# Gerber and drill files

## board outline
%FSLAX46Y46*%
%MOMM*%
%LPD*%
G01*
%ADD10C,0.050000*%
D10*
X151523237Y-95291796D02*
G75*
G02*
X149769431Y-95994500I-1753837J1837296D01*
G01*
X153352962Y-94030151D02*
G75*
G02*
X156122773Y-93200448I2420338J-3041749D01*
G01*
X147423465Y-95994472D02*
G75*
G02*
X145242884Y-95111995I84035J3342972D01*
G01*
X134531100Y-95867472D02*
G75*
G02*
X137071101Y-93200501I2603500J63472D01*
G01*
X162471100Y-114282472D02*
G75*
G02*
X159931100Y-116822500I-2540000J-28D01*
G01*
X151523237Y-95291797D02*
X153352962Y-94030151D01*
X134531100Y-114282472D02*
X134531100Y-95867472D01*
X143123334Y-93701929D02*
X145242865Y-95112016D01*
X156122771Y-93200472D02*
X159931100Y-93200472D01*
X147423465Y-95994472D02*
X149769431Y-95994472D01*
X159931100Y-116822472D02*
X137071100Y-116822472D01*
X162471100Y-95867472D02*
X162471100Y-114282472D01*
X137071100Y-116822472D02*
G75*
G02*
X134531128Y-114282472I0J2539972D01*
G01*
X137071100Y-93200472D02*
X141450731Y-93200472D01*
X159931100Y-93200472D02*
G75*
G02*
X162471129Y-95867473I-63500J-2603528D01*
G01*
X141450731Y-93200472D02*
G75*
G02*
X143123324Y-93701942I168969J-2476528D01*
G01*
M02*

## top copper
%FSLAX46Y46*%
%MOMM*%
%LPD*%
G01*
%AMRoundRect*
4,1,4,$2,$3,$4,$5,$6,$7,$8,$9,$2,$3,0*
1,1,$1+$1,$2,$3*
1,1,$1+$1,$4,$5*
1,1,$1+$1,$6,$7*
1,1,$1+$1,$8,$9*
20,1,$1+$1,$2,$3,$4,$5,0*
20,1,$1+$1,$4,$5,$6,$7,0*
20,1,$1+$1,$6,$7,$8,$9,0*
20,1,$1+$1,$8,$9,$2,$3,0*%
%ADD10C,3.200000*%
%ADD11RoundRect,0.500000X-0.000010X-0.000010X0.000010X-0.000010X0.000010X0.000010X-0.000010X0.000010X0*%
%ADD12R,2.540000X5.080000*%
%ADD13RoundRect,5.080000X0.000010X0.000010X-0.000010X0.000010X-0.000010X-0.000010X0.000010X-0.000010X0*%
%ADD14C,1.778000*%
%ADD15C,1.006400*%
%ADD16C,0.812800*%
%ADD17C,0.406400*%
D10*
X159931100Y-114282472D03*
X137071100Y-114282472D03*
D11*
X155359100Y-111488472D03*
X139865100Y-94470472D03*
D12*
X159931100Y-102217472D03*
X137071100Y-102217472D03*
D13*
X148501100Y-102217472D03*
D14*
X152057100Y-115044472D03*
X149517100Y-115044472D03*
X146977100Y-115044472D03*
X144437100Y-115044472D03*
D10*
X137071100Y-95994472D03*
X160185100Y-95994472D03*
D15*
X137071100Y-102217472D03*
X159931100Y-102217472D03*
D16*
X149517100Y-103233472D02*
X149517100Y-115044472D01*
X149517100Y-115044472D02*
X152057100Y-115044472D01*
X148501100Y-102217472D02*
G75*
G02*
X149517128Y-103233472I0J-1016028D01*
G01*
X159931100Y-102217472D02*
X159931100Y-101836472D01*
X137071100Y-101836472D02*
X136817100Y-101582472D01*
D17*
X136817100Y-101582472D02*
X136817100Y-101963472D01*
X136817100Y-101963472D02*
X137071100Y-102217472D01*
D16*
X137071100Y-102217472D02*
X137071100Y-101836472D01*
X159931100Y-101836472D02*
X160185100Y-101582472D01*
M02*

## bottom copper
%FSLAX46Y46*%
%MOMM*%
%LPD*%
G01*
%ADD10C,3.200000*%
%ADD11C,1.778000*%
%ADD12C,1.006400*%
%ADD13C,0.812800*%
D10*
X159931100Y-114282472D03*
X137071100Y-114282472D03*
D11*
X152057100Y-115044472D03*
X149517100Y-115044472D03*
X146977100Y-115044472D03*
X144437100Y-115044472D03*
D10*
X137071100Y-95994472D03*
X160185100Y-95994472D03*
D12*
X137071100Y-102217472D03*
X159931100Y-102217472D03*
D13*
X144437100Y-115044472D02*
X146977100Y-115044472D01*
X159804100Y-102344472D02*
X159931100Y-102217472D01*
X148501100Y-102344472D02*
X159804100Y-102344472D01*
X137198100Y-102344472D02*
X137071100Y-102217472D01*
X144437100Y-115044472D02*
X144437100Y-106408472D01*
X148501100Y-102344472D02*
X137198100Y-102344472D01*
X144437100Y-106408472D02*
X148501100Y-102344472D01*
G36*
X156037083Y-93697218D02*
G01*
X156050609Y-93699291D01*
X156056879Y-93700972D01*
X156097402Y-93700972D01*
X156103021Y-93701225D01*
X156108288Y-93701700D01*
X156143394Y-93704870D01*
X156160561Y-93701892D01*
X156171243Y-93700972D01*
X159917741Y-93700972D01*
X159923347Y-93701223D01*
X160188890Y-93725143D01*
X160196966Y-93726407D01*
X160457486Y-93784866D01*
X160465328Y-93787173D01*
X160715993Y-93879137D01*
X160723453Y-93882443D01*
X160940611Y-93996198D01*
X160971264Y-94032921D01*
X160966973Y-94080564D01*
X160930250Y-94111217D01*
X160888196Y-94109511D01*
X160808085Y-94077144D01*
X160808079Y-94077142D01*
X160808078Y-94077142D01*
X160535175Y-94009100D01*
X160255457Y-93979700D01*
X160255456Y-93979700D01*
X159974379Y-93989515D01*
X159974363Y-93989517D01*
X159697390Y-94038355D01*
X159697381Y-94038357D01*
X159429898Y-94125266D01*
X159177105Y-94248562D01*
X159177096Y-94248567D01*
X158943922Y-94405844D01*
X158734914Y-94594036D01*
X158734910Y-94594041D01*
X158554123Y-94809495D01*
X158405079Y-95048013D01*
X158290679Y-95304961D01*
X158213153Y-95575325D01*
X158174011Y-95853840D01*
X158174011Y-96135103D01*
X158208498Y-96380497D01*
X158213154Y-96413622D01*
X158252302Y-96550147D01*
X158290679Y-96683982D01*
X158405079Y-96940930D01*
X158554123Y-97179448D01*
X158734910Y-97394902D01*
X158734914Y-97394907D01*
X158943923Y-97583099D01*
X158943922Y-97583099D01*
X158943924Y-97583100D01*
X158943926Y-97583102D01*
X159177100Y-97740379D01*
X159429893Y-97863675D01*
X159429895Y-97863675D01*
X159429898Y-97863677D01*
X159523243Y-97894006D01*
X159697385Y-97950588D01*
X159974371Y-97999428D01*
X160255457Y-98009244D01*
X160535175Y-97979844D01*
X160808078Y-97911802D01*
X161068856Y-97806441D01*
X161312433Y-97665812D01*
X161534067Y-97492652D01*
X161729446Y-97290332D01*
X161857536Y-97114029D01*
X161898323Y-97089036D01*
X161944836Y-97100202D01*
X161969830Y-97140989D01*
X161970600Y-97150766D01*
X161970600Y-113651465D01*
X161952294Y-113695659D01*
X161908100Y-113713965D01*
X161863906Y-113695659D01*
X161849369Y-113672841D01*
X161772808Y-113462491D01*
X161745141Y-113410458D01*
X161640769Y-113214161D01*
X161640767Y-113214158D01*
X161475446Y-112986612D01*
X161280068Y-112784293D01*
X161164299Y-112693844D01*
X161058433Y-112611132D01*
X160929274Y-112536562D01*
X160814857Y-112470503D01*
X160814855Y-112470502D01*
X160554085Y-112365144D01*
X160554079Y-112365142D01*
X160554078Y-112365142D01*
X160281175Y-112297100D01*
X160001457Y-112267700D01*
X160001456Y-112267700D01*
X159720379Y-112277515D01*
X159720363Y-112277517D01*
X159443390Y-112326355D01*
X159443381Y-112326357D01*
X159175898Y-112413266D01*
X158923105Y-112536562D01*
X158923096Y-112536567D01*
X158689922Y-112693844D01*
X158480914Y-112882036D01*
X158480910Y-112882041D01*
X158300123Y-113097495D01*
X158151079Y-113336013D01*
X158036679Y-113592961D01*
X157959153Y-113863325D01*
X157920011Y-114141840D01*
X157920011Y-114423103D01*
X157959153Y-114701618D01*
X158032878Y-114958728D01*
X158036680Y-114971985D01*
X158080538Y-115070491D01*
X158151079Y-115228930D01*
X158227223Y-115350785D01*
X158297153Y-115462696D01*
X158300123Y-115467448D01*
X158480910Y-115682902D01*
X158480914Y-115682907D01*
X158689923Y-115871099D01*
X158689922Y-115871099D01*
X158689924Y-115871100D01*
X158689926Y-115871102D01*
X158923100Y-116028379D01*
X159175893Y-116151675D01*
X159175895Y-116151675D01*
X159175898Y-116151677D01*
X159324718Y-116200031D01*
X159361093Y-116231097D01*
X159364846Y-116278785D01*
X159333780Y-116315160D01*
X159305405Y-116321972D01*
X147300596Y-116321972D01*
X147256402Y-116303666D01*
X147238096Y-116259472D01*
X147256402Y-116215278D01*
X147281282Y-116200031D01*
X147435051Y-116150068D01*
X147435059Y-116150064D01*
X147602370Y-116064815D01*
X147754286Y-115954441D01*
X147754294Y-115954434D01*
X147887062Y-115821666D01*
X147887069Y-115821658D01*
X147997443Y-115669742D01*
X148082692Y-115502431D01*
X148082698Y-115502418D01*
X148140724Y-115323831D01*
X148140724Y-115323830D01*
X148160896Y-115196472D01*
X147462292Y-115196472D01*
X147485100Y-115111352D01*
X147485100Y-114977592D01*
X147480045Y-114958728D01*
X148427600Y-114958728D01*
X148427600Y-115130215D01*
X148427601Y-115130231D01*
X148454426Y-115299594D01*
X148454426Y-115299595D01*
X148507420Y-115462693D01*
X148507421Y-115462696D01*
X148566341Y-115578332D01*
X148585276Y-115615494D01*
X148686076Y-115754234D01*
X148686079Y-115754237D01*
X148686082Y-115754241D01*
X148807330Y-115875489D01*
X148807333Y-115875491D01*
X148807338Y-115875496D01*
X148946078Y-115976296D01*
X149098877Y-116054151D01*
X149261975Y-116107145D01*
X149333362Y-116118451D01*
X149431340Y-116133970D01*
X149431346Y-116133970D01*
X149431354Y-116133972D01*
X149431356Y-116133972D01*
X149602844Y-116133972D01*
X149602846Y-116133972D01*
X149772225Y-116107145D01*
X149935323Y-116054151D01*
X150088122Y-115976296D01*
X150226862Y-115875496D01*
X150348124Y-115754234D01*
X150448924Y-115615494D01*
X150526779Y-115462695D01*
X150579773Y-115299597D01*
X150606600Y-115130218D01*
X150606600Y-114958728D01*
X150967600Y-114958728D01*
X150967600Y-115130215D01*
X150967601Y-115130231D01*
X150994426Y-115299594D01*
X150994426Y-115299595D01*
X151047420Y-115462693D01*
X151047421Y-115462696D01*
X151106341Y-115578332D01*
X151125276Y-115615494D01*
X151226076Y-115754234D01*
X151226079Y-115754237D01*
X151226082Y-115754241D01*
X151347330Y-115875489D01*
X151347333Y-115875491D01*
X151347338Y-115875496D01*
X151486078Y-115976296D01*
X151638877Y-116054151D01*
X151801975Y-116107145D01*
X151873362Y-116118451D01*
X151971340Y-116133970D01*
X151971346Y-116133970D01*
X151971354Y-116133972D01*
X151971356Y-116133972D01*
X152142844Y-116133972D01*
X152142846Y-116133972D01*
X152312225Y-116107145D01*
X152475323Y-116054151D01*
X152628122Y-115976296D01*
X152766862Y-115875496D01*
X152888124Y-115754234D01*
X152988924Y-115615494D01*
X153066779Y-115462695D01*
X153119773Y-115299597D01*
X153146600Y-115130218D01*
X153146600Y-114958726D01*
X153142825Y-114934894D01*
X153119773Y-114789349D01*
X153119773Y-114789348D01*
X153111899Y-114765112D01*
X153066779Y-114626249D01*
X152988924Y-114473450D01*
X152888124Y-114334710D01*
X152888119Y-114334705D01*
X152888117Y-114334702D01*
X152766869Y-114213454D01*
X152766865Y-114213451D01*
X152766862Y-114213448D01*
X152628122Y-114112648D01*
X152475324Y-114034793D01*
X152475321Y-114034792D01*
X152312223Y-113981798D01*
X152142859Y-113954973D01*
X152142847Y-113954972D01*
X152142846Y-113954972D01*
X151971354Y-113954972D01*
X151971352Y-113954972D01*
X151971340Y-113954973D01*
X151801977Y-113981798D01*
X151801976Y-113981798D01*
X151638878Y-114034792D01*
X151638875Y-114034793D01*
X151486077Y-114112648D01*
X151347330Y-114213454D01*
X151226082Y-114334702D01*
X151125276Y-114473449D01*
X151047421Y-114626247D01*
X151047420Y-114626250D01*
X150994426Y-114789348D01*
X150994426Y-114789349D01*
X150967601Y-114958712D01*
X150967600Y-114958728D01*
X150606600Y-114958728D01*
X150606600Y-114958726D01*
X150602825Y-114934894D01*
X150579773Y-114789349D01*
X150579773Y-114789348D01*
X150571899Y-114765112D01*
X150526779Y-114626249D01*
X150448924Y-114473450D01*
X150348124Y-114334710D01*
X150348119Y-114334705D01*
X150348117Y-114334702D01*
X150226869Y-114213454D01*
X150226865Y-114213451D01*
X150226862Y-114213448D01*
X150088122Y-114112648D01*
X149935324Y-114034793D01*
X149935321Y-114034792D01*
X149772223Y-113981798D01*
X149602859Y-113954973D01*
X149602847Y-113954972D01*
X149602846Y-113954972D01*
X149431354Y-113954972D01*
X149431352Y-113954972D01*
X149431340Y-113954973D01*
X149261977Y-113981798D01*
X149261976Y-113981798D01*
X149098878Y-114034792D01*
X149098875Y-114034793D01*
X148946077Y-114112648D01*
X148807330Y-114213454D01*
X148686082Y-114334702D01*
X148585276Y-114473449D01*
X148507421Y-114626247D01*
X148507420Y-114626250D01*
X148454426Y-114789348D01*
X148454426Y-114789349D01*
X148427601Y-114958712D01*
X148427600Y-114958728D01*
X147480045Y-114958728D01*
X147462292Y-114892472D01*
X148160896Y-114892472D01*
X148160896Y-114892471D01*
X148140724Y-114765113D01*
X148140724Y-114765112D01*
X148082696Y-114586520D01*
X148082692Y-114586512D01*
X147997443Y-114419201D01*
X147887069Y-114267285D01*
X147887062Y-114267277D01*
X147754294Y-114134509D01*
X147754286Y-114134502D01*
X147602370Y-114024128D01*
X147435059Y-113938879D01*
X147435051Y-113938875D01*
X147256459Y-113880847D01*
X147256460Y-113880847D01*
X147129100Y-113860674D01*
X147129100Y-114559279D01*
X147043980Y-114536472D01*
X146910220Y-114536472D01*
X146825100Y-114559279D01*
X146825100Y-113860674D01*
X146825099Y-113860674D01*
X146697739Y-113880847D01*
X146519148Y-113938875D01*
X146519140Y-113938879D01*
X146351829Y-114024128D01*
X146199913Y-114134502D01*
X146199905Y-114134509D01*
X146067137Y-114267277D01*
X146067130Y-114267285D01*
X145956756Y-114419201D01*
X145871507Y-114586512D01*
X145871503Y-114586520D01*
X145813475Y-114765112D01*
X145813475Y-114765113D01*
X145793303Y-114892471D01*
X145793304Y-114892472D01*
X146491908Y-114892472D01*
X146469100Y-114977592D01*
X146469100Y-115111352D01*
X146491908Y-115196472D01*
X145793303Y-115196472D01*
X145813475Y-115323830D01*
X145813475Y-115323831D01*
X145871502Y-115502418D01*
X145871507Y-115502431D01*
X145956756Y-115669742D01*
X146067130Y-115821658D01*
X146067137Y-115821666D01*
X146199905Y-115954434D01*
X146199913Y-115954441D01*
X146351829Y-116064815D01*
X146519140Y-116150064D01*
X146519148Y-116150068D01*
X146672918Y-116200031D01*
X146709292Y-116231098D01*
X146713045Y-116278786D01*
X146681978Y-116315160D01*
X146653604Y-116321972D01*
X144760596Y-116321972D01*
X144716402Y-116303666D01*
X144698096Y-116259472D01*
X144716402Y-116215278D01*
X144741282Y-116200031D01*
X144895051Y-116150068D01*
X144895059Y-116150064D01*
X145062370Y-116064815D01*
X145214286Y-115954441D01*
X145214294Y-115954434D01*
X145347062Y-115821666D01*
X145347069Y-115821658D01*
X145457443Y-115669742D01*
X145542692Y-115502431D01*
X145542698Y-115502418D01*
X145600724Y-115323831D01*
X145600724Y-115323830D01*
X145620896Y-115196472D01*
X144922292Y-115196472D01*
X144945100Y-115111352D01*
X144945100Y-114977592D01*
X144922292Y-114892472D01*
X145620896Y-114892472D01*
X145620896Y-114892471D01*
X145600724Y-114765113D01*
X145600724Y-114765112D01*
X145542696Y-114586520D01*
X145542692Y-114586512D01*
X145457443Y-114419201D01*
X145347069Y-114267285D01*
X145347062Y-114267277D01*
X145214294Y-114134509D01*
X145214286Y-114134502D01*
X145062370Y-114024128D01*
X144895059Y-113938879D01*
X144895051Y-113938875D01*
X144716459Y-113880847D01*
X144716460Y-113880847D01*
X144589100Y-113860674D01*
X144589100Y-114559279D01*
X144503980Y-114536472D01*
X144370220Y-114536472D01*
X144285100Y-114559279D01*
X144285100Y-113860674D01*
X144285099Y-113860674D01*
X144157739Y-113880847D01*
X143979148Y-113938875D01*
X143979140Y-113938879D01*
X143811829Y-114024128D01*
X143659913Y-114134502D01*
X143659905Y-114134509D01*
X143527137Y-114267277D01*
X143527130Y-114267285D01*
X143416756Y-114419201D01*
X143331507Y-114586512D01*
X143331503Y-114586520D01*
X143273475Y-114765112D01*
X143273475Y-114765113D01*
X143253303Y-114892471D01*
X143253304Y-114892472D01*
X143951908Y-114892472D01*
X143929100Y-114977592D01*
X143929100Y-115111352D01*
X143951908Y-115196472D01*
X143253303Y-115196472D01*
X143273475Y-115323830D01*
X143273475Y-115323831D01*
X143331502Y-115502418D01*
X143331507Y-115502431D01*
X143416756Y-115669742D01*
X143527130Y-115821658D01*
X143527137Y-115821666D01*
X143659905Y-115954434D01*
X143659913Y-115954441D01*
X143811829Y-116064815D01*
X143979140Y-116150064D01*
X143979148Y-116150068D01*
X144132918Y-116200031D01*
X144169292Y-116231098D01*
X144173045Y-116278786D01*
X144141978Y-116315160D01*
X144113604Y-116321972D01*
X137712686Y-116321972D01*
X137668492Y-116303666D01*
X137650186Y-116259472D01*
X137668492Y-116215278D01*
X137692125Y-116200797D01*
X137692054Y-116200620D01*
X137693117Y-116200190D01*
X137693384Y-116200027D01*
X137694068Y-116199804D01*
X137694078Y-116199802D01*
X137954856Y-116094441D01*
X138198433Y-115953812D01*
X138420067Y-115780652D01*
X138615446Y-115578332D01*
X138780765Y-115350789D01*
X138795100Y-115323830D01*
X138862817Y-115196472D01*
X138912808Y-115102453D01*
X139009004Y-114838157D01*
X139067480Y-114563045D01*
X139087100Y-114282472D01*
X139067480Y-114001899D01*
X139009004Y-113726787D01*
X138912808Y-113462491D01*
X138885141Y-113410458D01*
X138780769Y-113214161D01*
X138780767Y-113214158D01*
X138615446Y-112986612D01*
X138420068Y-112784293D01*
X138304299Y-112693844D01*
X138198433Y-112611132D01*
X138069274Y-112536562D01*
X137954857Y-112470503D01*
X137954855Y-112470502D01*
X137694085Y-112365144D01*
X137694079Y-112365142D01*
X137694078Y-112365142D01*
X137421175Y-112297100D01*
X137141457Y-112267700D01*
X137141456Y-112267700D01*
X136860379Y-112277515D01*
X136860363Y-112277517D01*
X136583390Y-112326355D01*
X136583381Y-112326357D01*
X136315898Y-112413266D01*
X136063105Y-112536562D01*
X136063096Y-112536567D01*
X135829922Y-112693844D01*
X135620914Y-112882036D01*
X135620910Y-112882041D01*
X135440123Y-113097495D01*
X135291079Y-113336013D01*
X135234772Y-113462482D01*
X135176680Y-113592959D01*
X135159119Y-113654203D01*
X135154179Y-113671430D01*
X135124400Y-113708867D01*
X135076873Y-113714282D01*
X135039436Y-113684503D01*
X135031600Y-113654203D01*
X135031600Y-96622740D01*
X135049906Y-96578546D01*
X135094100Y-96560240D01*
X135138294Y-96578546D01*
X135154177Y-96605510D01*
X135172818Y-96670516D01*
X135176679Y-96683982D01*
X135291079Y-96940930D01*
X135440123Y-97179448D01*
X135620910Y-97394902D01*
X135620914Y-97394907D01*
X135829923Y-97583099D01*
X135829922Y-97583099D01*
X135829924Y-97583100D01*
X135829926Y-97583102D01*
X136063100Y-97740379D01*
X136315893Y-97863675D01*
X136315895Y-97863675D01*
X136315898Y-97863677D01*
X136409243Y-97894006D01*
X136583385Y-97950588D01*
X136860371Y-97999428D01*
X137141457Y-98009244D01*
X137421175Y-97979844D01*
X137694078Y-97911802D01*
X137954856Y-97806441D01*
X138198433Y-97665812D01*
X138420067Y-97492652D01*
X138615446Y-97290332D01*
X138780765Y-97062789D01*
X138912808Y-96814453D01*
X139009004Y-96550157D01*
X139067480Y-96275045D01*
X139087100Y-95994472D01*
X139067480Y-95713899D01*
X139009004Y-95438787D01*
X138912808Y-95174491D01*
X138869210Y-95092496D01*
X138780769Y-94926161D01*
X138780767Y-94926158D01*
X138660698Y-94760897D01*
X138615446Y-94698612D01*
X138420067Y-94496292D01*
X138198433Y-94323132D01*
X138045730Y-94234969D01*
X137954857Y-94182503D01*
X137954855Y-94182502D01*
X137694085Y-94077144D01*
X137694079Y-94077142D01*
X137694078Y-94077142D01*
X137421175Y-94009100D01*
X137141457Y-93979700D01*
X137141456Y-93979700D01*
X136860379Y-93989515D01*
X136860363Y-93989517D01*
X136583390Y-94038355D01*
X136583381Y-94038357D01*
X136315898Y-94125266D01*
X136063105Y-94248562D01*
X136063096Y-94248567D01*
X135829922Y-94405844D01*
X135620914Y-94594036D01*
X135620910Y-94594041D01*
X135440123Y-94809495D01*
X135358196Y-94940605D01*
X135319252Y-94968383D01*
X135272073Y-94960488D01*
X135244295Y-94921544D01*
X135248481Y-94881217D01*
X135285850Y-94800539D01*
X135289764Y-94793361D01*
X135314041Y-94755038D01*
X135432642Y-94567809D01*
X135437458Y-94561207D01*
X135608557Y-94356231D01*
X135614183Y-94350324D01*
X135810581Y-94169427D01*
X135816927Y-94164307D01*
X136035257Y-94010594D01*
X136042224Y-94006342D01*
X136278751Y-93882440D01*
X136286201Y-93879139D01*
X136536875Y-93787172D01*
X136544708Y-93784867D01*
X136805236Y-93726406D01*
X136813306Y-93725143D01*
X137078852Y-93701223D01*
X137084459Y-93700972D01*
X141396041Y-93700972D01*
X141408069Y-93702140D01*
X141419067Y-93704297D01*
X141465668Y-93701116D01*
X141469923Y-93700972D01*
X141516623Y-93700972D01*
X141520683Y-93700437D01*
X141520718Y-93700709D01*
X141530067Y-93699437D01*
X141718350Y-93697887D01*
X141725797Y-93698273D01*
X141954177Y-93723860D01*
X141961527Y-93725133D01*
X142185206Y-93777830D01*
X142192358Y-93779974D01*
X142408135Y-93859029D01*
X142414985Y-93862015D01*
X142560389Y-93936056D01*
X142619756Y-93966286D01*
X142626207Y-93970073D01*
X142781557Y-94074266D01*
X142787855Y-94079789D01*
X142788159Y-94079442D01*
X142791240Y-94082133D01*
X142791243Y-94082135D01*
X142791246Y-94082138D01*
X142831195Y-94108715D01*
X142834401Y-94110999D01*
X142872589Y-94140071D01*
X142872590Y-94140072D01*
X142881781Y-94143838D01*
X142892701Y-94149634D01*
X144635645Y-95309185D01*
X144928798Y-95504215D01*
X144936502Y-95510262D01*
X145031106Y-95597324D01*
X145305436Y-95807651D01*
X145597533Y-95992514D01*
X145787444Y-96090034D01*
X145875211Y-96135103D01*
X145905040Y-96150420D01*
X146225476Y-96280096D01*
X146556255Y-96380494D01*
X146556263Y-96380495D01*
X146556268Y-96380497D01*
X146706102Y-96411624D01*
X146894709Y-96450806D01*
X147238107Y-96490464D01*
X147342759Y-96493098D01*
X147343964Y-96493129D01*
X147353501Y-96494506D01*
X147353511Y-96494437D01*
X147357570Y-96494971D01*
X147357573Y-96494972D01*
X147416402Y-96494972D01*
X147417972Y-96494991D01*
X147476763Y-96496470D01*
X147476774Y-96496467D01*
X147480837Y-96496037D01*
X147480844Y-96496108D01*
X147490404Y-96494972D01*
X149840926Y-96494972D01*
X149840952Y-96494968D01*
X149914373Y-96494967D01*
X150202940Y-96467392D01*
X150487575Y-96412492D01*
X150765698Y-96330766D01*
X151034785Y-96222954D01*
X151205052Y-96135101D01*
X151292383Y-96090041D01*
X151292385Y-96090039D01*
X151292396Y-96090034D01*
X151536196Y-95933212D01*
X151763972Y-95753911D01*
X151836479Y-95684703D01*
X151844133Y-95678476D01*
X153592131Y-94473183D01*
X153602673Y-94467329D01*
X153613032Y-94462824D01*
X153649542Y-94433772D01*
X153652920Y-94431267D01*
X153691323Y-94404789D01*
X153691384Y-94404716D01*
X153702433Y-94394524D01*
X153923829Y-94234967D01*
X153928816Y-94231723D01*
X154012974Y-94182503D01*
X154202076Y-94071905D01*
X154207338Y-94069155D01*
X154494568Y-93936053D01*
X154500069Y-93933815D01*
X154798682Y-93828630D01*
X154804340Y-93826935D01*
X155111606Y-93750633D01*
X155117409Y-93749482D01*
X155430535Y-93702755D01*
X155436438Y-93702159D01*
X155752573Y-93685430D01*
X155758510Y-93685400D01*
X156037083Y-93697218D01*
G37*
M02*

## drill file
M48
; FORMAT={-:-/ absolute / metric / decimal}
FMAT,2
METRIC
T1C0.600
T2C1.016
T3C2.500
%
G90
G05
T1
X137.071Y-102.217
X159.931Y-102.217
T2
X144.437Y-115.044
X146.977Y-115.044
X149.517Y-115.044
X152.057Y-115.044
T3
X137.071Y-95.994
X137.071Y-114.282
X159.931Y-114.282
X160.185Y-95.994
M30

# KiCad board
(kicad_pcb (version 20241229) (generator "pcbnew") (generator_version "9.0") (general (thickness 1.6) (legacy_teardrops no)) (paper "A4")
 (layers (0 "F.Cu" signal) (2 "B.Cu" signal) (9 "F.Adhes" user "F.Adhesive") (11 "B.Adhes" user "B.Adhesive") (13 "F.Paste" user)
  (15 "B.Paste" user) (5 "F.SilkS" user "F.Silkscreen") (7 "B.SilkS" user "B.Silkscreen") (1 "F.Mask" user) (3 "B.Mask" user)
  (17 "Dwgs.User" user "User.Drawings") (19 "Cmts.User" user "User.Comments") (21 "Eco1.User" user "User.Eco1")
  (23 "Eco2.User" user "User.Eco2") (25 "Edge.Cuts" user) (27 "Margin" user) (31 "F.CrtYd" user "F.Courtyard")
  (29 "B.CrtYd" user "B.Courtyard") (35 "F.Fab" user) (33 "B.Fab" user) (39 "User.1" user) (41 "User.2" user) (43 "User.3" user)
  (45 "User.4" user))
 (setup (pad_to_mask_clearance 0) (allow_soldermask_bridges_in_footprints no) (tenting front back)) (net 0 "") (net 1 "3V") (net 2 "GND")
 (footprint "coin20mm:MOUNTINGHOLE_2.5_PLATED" (layer "F.Cu") (at 159.9311 114.282472)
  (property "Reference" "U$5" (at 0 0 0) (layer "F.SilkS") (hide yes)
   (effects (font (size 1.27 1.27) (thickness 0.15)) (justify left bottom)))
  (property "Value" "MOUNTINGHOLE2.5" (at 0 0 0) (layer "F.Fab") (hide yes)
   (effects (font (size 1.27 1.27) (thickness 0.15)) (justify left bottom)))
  (pad "P$1" thru_hole circle (at 0 0) (size 3.2 3.2) (drill 2.5) (layers "*.Cu" "*.Mask") (remove_unused_layers no)
   (solder_mask_margin 0.1016) (thermal_bridge_angle 0))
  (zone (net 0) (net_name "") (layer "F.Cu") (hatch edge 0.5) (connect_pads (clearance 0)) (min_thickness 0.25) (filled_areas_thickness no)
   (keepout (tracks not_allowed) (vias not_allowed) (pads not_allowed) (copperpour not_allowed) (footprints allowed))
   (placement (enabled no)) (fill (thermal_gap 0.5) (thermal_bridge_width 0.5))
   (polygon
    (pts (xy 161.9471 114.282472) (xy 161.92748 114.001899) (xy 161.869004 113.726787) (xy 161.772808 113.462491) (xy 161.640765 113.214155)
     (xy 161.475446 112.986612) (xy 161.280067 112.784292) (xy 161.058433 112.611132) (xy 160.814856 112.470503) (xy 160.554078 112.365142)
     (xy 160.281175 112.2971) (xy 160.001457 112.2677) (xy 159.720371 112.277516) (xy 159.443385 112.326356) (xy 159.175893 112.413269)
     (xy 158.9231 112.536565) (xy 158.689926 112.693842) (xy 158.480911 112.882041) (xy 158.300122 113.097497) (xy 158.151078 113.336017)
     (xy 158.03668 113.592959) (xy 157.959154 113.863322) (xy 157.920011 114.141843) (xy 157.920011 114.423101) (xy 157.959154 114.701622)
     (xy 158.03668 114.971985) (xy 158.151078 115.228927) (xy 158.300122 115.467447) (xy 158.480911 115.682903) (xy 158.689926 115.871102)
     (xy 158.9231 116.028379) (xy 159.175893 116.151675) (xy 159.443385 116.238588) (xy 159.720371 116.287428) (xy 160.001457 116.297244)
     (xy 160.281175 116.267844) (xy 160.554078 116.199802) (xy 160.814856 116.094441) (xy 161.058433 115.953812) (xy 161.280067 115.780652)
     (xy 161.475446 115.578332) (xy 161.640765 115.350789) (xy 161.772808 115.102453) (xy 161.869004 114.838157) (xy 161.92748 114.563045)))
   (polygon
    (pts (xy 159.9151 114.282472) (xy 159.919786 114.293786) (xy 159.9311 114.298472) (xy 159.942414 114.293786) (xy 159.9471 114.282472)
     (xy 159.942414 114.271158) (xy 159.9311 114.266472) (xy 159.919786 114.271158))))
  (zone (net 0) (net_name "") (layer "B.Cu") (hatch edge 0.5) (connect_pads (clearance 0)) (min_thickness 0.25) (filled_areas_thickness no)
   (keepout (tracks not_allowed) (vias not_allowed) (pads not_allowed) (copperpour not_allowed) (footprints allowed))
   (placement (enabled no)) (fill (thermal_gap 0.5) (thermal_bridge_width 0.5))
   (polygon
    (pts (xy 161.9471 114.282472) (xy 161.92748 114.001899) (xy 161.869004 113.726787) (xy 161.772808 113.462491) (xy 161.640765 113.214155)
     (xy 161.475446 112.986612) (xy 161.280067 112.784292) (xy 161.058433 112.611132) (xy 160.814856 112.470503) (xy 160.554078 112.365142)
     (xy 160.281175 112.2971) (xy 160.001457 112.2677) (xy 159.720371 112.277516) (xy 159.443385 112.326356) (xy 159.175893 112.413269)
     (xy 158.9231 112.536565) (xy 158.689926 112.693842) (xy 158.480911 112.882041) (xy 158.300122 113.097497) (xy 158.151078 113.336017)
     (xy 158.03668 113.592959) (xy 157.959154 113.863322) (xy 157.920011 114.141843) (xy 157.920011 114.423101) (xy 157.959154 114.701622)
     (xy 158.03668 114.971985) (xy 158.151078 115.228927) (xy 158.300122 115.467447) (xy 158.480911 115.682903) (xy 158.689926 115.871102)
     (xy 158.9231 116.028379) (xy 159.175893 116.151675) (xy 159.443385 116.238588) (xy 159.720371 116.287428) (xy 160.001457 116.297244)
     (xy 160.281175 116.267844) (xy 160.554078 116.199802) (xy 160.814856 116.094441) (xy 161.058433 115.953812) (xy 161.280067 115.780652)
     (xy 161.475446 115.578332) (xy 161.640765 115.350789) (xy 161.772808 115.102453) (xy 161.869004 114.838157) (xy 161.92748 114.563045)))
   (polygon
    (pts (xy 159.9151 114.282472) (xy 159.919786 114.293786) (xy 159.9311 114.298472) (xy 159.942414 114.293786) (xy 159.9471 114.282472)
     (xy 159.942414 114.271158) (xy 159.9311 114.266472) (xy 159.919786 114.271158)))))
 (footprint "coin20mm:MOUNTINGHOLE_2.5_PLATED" (layer "F.Cu") (at 137.0711 114.282472)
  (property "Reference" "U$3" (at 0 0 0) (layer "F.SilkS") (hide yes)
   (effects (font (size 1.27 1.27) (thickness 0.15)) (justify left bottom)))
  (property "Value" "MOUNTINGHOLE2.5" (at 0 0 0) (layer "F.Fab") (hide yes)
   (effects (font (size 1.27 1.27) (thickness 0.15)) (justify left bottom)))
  (pad "P$1" thru_hole circle (at 0 0) (size 3.2 3.2) (drill 2.5) (layers "*.Cu" "*.Mask") (remove_unused_layers no)
   (solder_mask_margin 0.1016) (thermal_bridge_angle 0))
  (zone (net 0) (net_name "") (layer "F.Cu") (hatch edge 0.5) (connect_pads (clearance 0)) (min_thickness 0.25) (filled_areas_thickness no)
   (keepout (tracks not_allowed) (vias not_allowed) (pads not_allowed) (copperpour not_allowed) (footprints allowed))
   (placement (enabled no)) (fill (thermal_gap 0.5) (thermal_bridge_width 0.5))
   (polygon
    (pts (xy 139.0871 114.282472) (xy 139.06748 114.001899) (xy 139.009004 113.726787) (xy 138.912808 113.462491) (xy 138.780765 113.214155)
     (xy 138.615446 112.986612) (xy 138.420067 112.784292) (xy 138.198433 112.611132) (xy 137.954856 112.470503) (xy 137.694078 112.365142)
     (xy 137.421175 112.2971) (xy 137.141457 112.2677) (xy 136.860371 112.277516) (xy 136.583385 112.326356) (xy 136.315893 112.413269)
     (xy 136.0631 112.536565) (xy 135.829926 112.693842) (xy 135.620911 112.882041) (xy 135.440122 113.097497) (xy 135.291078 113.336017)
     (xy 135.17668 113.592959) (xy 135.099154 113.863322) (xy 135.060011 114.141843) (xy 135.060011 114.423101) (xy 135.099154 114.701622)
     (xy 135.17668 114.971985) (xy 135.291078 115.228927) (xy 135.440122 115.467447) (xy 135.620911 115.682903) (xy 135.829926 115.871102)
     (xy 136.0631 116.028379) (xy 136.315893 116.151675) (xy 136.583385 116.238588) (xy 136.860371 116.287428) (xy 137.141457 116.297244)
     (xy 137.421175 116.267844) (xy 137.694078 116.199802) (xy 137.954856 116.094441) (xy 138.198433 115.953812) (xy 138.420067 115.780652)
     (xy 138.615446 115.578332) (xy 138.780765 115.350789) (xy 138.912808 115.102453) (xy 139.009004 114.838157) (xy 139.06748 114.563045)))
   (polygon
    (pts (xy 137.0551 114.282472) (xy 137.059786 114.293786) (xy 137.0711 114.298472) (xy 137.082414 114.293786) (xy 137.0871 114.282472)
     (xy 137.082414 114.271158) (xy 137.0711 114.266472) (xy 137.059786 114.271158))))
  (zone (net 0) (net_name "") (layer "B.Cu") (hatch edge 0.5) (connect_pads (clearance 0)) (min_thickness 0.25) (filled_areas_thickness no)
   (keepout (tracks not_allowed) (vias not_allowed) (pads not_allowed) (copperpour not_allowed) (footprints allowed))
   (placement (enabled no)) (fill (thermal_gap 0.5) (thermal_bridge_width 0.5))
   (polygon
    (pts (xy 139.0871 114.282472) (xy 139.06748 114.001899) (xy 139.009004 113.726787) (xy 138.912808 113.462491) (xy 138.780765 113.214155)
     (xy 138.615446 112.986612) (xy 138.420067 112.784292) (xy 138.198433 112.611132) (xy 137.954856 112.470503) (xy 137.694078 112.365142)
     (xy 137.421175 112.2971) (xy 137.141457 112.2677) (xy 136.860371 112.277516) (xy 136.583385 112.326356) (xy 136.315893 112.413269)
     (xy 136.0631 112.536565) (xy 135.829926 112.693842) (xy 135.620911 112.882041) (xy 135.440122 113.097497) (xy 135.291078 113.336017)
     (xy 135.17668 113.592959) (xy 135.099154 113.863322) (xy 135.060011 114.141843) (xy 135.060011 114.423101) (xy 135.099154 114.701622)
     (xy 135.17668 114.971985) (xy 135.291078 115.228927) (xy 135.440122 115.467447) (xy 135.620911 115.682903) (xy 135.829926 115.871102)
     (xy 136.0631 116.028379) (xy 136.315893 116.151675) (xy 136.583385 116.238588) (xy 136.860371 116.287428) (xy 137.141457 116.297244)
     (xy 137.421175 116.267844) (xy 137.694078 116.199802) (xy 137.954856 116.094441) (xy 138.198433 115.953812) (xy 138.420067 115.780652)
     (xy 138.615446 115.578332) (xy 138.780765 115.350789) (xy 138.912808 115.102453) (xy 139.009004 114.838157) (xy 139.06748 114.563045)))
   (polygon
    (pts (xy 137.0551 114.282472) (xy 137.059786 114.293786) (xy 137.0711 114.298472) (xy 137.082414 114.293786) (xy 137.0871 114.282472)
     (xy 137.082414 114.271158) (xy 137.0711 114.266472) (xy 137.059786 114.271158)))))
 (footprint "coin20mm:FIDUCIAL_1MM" (layer "F.Cu") (at 155.3591 111.488472)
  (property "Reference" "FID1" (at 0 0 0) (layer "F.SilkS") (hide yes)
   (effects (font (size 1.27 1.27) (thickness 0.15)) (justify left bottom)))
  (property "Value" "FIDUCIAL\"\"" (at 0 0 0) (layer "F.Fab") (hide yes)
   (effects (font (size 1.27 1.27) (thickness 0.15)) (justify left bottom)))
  (pad "1" smd roundrect (at 0 0) (size 1 1) (layers "F.Cu" "F.Mask") (roundrect_rratio 0.5) (solder_mask_margin 0.1016)
   (solder_paste_margin 0) (thermal_bridge_angle 0)))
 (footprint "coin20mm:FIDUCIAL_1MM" (layer "F.Cu") (at 139.8651 94.470472)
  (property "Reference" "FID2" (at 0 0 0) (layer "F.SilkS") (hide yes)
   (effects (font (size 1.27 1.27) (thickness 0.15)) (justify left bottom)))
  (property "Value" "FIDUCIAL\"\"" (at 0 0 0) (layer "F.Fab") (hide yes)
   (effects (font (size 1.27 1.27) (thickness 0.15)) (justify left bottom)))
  (pad "1" smd roundrect (at 0 0) (size 1 1) (layers "F.Cu" "F.Mask") (roundrect_rratio 0.5) (solder_mask_margin 0.1016)
   (solder_paste_margin 0) (thermal_bridge_angle 0)))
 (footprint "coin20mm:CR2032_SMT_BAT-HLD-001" (layer "F.Cu") (at 148.5011 102.217472 180)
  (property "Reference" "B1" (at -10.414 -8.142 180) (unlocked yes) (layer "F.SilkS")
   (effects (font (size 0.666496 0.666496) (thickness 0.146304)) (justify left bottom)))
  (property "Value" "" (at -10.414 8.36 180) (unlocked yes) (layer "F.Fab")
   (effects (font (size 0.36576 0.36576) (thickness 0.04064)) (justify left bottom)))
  (pad "+$1" smd rect (at -11.43 0 180) (size 2.54 5.08) (layers "F.Cu" "F.Mask" "F.Paste") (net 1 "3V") (solder_mask_margin 0.1016)
   (solder_paste_margin 0) (thermal_bridge_angle 0))
  (pad "+$2" smd rect (at 11.43 0 180) (size 2.54 5.08) (layers "F.Cu" "F.Mask" "F.Paste") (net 1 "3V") (solder_mask_margin 0.1016)
   (solder_paste_margin 0) (thermal_bridge_angle 0))
  (pad "-" smd roundrect (at 0 0 180) (size 10.16 10.16) (layers "F.Cu" "F.Mask") (roundrect_rratio 0.5) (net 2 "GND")
   (solder_mask_margin 0.1016) (solder_paste_margin 0) (thermal_bridge_angle 0)))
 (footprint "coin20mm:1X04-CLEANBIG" (layer "F.Cu") (at 148.2471 115.044472 180)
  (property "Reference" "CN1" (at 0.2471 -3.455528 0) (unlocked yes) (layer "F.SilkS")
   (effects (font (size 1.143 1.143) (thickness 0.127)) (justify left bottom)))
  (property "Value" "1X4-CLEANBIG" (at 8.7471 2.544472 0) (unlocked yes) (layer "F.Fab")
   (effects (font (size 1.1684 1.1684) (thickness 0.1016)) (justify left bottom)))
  (pad "1" thru_hole circle (at -3.81 0 270) (size 1.778 1.778) (drill 1.016) (layers "*.Cu" "*.Mask") (remove_unused_layers no)
   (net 2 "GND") (solder_mask_margin 0.1016) (thermal_bridge_angle 0))
  (pad "2" thru_hole circle (at -1.27 0 270) (size 1.778 1.778) (drill 1.016) (layers "*.Cu" "*.Mask") (remove_unused_layers no)
   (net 2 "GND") (solder_mask_margin 0.1016) (thermal_bridge_angle 0))
  (pad "3" thru_hole circle (at 1.27 0 270) (size 1.778 1.778) (drill 1.016) (layers "*.Cu" "*.Mask") (remove_unused_layers no) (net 1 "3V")
   (solder_mask_margin 0.1016) (thermal_bridge_angle 0))
  (pad "4" thru_hole circle (at 3.81 0 270) (size 1.778 1.778) (drill 1.016) (layers "*.Cu" "*.Mask") (remove_unused_layers no) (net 1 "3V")
   (solder_mask_margin 0.1016) (thermal_bridge_angle 0)))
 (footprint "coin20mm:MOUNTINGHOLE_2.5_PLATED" (layer "F.Cu") (at 137.0711 95.994472)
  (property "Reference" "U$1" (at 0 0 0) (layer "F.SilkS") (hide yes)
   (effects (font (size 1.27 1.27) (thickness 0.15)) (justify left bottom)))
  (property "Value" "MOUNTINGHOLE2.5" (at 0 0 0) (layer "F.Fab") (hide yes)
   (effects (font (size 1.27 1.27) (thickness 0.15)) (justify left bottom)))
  (pad "P$1" thru_hole circle (at 0 0) (size 3.2 3.2) (drill 2.5) (layers "*.Cu" "*.Mask") (remove_unused_layers no)
   (solder_mask_margin 0.1016) (thermal_bridge_angle 0))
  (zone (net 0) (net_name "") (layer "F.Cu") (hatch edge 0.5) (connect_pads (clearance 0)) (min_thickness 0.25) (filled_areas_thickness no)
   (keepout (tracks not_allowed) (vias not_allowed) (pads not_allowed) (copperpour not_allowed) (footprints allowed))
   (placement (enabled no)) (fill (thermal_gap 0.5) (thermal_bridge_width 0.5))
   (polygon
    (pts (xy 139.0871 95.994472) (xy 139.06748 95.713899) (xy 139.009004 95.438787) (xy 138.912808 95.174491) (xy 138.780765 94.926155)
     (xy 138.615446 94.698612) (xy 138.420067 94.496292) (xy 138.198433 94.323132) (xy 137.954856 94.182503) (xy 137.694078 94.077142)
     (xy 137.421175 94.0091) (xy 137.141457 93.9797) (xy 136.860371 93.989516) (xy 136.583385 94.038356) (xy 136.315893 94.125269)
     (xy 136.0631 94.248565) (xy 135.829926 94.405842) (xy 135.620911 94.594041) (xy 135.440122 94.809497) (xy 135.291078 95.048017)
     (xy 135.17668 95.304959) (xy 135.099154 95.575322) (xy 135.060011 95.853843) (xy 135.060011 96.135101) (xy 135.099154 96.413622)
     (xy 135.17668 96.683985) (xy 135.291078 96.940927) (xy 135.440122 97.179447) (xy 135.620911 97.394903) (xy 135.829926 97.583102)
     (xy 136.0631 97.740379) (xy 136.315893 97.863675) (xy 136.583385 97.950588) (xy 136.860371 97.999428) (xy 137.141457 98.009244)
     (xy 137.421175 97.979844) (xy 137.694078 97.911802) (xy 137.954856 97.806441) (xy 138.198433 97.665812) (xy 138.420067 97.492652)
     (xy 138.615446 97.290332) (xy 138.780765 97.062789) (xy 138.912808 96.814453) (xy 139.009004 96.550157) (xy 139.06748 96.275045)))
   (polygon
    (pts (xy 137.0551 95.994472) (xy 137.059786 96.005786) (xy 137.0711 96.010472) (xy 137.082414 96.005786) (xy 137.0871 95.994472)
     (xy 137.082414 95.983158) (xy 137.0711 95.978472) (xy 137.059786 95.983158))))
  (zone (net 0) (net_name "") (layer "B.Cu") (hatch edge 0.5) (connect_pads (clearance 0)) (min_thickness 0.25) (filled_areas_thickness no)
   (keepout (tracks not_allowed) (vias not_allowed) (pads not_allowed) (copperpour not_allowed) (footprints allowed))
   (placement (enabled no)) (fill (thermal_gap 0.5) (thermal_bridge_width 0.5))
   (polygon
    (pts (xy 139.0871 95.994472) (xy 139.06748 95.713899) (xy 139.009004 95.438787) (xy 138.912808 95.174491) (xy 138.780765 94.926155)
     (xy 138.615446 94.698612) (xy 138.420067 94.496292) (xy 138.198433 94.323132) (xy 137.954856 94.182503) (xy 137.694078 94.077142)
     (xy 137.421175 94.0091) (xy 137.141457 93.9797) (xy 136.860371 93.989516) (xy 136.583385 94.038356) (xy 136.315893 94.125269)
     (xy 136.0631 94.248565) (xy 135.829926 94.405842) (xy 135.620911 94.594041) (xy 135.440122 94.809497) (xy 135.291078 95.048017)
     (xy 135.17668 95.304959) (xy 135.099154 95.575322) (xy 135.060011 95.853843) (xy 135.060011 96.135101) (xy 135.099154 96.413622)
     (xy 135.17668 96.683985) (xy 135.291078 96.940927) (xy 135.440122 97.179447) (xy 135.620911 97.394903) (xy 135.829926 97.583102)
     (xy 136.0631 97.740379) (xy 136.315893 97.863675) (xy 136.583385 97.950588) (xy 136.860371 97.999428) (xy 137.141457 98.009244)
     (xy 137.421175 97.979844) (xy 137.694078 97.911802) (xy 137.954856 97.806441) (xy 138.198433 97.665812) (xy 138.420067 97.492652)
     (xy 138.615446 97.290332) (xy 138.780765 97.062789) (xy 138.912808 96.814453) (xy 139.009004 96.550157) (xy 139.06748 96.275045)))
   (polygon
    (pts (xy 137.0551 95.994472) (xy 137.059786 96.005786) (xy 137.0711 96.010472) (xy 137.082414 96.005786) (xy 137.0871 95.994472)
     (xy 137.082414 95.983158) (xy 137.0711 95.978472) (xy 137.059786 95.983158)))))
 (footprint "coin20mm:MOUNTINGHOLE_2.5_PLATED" (layer "F.Cu") (at 160.1851 95.994472)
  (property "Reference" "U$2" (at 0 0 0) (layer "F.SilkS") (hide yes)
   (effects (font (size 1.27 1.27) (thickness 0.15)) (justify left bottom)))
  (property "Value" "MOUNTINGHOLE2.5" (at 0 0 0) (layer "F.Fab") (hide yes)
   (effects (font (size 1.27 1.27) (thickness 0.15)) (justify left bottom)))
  (pad "P$1" thru_hole circle (at 0 0) (size 3.2 3.2) (drill 2.5) (layers "*.Cu" "*.Mask") (remove_unused_layers no)
   (solder_mask_margin 0.1016) (thermal_bridge_angle 0))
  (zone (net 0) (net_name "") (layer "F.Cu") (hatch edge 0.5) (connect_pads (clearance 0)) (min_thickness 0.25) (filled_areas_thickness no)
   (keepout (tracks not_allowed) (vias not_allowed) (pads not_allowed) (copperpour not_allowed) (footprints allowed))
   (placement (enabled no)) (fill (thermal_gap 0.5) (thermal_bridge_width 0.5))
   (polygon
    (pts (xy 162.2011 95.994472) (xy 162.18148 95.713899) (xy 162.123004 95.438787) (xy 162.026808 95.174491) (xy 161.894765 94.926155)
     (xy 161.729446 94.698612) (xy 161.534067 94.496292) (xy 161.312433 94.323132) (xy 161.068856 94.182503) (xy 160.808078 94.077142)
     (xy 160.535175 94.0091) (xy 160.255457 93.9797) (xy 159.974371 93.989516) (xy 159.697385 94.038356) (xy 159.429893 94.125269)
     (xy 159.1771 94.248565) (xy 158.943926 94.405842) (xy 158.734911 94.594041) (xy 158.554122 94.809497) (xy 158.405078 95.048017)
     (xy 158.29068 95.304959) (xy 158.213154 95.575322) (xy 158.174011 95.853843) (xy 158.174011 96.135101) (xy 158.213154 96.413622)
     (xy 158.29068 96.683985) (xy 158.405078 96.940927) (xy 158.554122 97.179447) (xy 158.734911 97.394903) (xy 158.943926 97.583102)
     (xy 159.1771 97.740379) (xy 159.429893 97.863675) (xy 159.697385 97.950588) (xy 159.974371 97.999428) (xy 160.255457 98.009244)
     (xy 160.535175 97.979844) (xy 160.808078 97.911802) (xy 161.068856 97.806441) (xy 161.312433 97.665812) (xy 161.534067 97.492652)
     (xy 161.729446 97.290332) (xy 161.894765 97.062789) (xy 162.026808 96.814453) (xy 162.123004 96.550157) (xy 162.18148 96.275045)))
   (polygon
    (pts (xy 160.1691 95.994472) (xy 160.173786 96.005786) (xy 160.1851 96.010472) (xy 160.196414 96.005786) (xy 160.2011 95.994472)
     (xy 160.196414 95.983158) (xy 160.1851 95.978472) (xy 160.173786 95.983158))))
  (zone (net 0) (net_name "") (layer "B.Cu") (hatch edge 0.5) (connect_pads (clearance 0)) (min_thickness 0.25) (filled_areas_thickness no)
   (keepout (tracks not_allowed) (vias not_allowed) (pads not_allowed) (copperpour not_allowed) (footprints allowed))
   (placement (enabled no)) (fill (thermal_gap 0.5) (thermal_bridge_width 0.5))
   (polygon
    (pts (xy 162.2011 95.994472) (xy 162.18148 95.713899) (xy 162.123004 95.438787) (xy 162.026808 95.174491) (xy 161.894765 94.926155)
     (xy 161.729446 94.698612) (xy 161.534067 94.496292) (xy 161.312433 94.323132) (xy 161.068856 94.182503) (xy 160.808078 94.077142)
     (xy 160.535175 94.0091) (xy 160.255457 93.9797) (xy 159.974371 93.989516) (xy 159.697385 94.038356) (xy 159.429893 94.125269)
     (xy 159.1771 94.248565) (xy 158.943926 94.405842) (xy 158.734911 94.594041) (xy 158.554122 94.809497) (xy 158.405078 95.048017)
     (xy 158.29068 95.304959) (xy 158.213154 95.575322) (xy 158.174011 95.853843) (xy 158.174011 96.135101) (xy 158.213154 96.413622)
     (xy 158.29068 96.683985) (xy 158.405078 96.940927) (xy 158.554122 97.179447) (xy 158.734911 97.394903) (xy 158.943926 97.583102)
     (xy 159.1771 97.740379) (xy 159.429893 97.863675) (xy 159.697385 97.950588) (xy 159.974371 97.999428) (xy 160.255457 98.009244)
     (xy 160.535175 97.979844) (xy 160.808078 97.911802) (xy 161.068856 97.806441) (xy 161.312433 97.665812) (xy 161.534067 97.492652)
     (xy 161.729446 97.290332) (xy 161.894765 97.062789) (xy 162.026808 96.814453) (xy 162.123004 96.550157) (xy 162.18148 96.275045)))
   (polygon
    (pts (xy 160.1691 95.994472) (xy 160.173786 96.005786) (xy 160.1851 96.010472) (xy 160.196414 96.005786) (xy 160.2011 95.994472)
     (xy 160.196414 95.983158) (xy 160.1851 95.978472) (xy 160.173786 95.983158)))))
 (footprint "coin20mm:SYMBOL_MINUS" (layer "F.Cu") (at 154.2161 115.044472)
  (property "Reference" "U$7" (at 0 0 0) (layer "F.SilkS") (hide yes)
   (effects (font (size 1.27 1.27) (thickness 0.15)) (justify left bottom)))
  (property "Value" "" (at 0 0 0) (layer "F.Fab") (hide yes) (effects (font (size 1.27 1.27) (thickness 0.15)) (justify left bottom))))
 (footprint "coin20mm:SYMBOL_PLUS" (layer "F.Cu") (at 142.2781 115.044472)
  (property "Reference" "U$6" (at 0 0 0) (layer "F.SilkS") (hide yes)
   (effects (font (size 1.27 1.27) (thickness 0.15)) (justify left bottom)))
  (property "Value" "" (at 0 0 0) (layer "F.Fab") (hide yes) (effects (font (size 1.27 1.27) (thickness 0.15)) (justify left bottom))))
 (gr_arc (start 151.523237 95.291796) (mid 150.714099 95.812267) (end 149.769431 95.994472) (stroke (width 0.05) (type solid))
  (layer "Edge.Cuts"))
 (gr_arc (start 153.352962 94.030151) (mid 154.657854 93.348196) (end 156.122771 93.200472) (stroke (width 0.05) (type solid))
  (layer "Edge.Cuts"))
 (gr_arc (start 147.423465 95.994472) (mid 146.253008 95.751316) (end 145.242865 95.112016) (stroke (width 0.05) (type solid))
  (layer "Edge.Cuts"))
 (gr_arc (start 134.5311 95.867472) (mid 135.248746 94.007921) (end 137.0711 93.200472) (stroke (width 0.05) (type solid))
  (layer "Edge.Cuts"))
 (gr_arc (start 162.4711 114.282472) (mid 161.727151 116.078523) (end 159.9311 116.822472) (stroke (width 0.05) (type solid))
  (layer "Edge.Cuts"))
 (gr_line (start 151.523237 95.291797) (end 153.352962 94.030151) (stroke (width 0.05) (type solid)) (layer "Edge.Cuts"))
 (gr_line (start 134.5311 114.282472) (end 134.5311 95.867472) (stroke (width 0.05) (type solid)) (layer "Edge.Cuts"))
 (gr_line (start 143.123334 93.701929) (end 145.242865 95.112016) (stroke (width 0.05) (type solid)) (layer "Edge.Cuts"))
 (gr_line (start 156.122771 93.200472) (end 159.9311 93.200472) (stroke (width 0.05) (type solid)) (layer "Edge.Cuts"))
 (gr_line (start 147.423465 95.994472) (end 149.769431 95.994472) (stroke (width 0.05) (type solid)) (layer "Edge.Cuts"))
 (gr_line (start 159.9311 116.822472) (end 137.0711 116.822472) (stroke (width 0.05) (type solid)) (layer "Edge.Cuts"))
 (gr_line (start 162.4711 95.867472) (end 162.4711 114.282472) (stroke (width 0.05) (type solid)) (layer "Edge.Cuts"))
 (gr_arc (start 137.0711 116.822472) (mid 135.275049 116.078523) (end 134.5311 114.282472) (stroke (width 0.05) (type solid))
  (layer "Edge.Cuts"))
 (gr_line (start 137.0711 93.200472) (end 141.450731 93.200472) (stroke (width 0.05) (type solid)) (layer "Edge.Cuts"))
 (gr_arc (start 159.9311 93.200472) (mid 161.753454 94.007921) (end 162.4711 95.867472) (stroke (width 0.05) (type solid))
  (layer "Edge.Cuts"))
 (gr_arc (start 141.450731 93.200472) (mid 142.332582 93.299272) (end 143.123334 93.701929) (stroke (width 0.05) (type solid))
  (layer "Edge.Cuts"))
 (segment (start 149.5171 103.233472) (end 149.5171 115.044472) (width 0.8128) (layer "F.Cu") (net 2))
 (segment (start 149.5171 115.044472) (end 152.0571 115.044472) (width 0.8128) (layer "F.Cu") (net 2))
 (arc (start 148.5011 102.217472) (mid 149.21952 102.515052) (end 149.5171 103.233472) (width 0.8128) (layer "F.Cu") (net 2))
 (segment (start 159.9311 102.217472) (end 159.9311 101.836472) (width 0.8128) (layer "F.Cu") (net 1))
 (segment (start 137.0711 101.836472) (end 136.8171 101.582472) (width 0.8128) (layer "F.Cu") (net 1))
 (segment (start 136.8171 101.582472) (end 136.8171 101.963472) (width 0.4064) (layer "F.Cu") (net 1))
 (segment (start 136.8171 101.963472) (end 137.0711 102.217472) (width 0.4064) (layer "F.Cu") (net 1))
 (segment (start 137.0711 102.217472) (end 137.0711 101.836472) (width 0.8128) (layer "F.Cu") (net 1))
 (segment (start 159.9311 101.836472) (end 160.1851 101.582472) (width 0.8128) (layer "F.Cu") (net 1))
 (via (at 137.0711 102.217472) (size 1.0064) (drill 0.6) (layers "F.Cu" "B.Cu") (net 1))
 (via (at 159.9311 102.217472) (size 1.0064) (drill 0.6) (layers "F.Cu" "B.Cu") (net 1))
 (segment (start 144.4371 115.044472) (end 146.9771 115.044472) (width 0.8128) (layer "B.Cu") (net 1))
 (segment (start 159.8041 102.344472) (end 159.9311 102.217472) (width 0.8128) (layer "B.Cu") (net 1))
 (segment (start 148.5011 102.344472) (end 159.8041 102.344472) (width 0.8128) (layer "B.Cu") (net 1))
 (segment (start 137.1981 102.344472) (end 137.0711 102.217472) (width 0.8128) (layer "B.Cu") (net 1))
 (segment (start 144.4371 115.044472) (end 144.4371 106.408472) (width 0.8128) (layer "B.Cu") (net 1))
 (segment (start 148.5011 102.344472) (end 137.1981 102.344472) (width 0.8128) (layer "B.Cu") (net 1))
 (segment (start 144.4371 106.408472) (end 148.5011 102.344472) (width 0.8128) (layer "B.Cu") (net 1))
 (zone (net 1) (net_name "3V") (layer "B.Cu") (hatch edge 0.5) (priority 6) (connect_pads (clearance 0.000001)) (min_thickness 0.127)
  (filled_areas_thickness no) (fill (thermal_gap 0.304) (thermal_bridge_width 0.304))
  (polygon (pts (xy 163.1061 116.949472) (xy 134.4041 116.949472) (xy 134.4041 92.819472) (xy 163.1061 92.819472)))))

